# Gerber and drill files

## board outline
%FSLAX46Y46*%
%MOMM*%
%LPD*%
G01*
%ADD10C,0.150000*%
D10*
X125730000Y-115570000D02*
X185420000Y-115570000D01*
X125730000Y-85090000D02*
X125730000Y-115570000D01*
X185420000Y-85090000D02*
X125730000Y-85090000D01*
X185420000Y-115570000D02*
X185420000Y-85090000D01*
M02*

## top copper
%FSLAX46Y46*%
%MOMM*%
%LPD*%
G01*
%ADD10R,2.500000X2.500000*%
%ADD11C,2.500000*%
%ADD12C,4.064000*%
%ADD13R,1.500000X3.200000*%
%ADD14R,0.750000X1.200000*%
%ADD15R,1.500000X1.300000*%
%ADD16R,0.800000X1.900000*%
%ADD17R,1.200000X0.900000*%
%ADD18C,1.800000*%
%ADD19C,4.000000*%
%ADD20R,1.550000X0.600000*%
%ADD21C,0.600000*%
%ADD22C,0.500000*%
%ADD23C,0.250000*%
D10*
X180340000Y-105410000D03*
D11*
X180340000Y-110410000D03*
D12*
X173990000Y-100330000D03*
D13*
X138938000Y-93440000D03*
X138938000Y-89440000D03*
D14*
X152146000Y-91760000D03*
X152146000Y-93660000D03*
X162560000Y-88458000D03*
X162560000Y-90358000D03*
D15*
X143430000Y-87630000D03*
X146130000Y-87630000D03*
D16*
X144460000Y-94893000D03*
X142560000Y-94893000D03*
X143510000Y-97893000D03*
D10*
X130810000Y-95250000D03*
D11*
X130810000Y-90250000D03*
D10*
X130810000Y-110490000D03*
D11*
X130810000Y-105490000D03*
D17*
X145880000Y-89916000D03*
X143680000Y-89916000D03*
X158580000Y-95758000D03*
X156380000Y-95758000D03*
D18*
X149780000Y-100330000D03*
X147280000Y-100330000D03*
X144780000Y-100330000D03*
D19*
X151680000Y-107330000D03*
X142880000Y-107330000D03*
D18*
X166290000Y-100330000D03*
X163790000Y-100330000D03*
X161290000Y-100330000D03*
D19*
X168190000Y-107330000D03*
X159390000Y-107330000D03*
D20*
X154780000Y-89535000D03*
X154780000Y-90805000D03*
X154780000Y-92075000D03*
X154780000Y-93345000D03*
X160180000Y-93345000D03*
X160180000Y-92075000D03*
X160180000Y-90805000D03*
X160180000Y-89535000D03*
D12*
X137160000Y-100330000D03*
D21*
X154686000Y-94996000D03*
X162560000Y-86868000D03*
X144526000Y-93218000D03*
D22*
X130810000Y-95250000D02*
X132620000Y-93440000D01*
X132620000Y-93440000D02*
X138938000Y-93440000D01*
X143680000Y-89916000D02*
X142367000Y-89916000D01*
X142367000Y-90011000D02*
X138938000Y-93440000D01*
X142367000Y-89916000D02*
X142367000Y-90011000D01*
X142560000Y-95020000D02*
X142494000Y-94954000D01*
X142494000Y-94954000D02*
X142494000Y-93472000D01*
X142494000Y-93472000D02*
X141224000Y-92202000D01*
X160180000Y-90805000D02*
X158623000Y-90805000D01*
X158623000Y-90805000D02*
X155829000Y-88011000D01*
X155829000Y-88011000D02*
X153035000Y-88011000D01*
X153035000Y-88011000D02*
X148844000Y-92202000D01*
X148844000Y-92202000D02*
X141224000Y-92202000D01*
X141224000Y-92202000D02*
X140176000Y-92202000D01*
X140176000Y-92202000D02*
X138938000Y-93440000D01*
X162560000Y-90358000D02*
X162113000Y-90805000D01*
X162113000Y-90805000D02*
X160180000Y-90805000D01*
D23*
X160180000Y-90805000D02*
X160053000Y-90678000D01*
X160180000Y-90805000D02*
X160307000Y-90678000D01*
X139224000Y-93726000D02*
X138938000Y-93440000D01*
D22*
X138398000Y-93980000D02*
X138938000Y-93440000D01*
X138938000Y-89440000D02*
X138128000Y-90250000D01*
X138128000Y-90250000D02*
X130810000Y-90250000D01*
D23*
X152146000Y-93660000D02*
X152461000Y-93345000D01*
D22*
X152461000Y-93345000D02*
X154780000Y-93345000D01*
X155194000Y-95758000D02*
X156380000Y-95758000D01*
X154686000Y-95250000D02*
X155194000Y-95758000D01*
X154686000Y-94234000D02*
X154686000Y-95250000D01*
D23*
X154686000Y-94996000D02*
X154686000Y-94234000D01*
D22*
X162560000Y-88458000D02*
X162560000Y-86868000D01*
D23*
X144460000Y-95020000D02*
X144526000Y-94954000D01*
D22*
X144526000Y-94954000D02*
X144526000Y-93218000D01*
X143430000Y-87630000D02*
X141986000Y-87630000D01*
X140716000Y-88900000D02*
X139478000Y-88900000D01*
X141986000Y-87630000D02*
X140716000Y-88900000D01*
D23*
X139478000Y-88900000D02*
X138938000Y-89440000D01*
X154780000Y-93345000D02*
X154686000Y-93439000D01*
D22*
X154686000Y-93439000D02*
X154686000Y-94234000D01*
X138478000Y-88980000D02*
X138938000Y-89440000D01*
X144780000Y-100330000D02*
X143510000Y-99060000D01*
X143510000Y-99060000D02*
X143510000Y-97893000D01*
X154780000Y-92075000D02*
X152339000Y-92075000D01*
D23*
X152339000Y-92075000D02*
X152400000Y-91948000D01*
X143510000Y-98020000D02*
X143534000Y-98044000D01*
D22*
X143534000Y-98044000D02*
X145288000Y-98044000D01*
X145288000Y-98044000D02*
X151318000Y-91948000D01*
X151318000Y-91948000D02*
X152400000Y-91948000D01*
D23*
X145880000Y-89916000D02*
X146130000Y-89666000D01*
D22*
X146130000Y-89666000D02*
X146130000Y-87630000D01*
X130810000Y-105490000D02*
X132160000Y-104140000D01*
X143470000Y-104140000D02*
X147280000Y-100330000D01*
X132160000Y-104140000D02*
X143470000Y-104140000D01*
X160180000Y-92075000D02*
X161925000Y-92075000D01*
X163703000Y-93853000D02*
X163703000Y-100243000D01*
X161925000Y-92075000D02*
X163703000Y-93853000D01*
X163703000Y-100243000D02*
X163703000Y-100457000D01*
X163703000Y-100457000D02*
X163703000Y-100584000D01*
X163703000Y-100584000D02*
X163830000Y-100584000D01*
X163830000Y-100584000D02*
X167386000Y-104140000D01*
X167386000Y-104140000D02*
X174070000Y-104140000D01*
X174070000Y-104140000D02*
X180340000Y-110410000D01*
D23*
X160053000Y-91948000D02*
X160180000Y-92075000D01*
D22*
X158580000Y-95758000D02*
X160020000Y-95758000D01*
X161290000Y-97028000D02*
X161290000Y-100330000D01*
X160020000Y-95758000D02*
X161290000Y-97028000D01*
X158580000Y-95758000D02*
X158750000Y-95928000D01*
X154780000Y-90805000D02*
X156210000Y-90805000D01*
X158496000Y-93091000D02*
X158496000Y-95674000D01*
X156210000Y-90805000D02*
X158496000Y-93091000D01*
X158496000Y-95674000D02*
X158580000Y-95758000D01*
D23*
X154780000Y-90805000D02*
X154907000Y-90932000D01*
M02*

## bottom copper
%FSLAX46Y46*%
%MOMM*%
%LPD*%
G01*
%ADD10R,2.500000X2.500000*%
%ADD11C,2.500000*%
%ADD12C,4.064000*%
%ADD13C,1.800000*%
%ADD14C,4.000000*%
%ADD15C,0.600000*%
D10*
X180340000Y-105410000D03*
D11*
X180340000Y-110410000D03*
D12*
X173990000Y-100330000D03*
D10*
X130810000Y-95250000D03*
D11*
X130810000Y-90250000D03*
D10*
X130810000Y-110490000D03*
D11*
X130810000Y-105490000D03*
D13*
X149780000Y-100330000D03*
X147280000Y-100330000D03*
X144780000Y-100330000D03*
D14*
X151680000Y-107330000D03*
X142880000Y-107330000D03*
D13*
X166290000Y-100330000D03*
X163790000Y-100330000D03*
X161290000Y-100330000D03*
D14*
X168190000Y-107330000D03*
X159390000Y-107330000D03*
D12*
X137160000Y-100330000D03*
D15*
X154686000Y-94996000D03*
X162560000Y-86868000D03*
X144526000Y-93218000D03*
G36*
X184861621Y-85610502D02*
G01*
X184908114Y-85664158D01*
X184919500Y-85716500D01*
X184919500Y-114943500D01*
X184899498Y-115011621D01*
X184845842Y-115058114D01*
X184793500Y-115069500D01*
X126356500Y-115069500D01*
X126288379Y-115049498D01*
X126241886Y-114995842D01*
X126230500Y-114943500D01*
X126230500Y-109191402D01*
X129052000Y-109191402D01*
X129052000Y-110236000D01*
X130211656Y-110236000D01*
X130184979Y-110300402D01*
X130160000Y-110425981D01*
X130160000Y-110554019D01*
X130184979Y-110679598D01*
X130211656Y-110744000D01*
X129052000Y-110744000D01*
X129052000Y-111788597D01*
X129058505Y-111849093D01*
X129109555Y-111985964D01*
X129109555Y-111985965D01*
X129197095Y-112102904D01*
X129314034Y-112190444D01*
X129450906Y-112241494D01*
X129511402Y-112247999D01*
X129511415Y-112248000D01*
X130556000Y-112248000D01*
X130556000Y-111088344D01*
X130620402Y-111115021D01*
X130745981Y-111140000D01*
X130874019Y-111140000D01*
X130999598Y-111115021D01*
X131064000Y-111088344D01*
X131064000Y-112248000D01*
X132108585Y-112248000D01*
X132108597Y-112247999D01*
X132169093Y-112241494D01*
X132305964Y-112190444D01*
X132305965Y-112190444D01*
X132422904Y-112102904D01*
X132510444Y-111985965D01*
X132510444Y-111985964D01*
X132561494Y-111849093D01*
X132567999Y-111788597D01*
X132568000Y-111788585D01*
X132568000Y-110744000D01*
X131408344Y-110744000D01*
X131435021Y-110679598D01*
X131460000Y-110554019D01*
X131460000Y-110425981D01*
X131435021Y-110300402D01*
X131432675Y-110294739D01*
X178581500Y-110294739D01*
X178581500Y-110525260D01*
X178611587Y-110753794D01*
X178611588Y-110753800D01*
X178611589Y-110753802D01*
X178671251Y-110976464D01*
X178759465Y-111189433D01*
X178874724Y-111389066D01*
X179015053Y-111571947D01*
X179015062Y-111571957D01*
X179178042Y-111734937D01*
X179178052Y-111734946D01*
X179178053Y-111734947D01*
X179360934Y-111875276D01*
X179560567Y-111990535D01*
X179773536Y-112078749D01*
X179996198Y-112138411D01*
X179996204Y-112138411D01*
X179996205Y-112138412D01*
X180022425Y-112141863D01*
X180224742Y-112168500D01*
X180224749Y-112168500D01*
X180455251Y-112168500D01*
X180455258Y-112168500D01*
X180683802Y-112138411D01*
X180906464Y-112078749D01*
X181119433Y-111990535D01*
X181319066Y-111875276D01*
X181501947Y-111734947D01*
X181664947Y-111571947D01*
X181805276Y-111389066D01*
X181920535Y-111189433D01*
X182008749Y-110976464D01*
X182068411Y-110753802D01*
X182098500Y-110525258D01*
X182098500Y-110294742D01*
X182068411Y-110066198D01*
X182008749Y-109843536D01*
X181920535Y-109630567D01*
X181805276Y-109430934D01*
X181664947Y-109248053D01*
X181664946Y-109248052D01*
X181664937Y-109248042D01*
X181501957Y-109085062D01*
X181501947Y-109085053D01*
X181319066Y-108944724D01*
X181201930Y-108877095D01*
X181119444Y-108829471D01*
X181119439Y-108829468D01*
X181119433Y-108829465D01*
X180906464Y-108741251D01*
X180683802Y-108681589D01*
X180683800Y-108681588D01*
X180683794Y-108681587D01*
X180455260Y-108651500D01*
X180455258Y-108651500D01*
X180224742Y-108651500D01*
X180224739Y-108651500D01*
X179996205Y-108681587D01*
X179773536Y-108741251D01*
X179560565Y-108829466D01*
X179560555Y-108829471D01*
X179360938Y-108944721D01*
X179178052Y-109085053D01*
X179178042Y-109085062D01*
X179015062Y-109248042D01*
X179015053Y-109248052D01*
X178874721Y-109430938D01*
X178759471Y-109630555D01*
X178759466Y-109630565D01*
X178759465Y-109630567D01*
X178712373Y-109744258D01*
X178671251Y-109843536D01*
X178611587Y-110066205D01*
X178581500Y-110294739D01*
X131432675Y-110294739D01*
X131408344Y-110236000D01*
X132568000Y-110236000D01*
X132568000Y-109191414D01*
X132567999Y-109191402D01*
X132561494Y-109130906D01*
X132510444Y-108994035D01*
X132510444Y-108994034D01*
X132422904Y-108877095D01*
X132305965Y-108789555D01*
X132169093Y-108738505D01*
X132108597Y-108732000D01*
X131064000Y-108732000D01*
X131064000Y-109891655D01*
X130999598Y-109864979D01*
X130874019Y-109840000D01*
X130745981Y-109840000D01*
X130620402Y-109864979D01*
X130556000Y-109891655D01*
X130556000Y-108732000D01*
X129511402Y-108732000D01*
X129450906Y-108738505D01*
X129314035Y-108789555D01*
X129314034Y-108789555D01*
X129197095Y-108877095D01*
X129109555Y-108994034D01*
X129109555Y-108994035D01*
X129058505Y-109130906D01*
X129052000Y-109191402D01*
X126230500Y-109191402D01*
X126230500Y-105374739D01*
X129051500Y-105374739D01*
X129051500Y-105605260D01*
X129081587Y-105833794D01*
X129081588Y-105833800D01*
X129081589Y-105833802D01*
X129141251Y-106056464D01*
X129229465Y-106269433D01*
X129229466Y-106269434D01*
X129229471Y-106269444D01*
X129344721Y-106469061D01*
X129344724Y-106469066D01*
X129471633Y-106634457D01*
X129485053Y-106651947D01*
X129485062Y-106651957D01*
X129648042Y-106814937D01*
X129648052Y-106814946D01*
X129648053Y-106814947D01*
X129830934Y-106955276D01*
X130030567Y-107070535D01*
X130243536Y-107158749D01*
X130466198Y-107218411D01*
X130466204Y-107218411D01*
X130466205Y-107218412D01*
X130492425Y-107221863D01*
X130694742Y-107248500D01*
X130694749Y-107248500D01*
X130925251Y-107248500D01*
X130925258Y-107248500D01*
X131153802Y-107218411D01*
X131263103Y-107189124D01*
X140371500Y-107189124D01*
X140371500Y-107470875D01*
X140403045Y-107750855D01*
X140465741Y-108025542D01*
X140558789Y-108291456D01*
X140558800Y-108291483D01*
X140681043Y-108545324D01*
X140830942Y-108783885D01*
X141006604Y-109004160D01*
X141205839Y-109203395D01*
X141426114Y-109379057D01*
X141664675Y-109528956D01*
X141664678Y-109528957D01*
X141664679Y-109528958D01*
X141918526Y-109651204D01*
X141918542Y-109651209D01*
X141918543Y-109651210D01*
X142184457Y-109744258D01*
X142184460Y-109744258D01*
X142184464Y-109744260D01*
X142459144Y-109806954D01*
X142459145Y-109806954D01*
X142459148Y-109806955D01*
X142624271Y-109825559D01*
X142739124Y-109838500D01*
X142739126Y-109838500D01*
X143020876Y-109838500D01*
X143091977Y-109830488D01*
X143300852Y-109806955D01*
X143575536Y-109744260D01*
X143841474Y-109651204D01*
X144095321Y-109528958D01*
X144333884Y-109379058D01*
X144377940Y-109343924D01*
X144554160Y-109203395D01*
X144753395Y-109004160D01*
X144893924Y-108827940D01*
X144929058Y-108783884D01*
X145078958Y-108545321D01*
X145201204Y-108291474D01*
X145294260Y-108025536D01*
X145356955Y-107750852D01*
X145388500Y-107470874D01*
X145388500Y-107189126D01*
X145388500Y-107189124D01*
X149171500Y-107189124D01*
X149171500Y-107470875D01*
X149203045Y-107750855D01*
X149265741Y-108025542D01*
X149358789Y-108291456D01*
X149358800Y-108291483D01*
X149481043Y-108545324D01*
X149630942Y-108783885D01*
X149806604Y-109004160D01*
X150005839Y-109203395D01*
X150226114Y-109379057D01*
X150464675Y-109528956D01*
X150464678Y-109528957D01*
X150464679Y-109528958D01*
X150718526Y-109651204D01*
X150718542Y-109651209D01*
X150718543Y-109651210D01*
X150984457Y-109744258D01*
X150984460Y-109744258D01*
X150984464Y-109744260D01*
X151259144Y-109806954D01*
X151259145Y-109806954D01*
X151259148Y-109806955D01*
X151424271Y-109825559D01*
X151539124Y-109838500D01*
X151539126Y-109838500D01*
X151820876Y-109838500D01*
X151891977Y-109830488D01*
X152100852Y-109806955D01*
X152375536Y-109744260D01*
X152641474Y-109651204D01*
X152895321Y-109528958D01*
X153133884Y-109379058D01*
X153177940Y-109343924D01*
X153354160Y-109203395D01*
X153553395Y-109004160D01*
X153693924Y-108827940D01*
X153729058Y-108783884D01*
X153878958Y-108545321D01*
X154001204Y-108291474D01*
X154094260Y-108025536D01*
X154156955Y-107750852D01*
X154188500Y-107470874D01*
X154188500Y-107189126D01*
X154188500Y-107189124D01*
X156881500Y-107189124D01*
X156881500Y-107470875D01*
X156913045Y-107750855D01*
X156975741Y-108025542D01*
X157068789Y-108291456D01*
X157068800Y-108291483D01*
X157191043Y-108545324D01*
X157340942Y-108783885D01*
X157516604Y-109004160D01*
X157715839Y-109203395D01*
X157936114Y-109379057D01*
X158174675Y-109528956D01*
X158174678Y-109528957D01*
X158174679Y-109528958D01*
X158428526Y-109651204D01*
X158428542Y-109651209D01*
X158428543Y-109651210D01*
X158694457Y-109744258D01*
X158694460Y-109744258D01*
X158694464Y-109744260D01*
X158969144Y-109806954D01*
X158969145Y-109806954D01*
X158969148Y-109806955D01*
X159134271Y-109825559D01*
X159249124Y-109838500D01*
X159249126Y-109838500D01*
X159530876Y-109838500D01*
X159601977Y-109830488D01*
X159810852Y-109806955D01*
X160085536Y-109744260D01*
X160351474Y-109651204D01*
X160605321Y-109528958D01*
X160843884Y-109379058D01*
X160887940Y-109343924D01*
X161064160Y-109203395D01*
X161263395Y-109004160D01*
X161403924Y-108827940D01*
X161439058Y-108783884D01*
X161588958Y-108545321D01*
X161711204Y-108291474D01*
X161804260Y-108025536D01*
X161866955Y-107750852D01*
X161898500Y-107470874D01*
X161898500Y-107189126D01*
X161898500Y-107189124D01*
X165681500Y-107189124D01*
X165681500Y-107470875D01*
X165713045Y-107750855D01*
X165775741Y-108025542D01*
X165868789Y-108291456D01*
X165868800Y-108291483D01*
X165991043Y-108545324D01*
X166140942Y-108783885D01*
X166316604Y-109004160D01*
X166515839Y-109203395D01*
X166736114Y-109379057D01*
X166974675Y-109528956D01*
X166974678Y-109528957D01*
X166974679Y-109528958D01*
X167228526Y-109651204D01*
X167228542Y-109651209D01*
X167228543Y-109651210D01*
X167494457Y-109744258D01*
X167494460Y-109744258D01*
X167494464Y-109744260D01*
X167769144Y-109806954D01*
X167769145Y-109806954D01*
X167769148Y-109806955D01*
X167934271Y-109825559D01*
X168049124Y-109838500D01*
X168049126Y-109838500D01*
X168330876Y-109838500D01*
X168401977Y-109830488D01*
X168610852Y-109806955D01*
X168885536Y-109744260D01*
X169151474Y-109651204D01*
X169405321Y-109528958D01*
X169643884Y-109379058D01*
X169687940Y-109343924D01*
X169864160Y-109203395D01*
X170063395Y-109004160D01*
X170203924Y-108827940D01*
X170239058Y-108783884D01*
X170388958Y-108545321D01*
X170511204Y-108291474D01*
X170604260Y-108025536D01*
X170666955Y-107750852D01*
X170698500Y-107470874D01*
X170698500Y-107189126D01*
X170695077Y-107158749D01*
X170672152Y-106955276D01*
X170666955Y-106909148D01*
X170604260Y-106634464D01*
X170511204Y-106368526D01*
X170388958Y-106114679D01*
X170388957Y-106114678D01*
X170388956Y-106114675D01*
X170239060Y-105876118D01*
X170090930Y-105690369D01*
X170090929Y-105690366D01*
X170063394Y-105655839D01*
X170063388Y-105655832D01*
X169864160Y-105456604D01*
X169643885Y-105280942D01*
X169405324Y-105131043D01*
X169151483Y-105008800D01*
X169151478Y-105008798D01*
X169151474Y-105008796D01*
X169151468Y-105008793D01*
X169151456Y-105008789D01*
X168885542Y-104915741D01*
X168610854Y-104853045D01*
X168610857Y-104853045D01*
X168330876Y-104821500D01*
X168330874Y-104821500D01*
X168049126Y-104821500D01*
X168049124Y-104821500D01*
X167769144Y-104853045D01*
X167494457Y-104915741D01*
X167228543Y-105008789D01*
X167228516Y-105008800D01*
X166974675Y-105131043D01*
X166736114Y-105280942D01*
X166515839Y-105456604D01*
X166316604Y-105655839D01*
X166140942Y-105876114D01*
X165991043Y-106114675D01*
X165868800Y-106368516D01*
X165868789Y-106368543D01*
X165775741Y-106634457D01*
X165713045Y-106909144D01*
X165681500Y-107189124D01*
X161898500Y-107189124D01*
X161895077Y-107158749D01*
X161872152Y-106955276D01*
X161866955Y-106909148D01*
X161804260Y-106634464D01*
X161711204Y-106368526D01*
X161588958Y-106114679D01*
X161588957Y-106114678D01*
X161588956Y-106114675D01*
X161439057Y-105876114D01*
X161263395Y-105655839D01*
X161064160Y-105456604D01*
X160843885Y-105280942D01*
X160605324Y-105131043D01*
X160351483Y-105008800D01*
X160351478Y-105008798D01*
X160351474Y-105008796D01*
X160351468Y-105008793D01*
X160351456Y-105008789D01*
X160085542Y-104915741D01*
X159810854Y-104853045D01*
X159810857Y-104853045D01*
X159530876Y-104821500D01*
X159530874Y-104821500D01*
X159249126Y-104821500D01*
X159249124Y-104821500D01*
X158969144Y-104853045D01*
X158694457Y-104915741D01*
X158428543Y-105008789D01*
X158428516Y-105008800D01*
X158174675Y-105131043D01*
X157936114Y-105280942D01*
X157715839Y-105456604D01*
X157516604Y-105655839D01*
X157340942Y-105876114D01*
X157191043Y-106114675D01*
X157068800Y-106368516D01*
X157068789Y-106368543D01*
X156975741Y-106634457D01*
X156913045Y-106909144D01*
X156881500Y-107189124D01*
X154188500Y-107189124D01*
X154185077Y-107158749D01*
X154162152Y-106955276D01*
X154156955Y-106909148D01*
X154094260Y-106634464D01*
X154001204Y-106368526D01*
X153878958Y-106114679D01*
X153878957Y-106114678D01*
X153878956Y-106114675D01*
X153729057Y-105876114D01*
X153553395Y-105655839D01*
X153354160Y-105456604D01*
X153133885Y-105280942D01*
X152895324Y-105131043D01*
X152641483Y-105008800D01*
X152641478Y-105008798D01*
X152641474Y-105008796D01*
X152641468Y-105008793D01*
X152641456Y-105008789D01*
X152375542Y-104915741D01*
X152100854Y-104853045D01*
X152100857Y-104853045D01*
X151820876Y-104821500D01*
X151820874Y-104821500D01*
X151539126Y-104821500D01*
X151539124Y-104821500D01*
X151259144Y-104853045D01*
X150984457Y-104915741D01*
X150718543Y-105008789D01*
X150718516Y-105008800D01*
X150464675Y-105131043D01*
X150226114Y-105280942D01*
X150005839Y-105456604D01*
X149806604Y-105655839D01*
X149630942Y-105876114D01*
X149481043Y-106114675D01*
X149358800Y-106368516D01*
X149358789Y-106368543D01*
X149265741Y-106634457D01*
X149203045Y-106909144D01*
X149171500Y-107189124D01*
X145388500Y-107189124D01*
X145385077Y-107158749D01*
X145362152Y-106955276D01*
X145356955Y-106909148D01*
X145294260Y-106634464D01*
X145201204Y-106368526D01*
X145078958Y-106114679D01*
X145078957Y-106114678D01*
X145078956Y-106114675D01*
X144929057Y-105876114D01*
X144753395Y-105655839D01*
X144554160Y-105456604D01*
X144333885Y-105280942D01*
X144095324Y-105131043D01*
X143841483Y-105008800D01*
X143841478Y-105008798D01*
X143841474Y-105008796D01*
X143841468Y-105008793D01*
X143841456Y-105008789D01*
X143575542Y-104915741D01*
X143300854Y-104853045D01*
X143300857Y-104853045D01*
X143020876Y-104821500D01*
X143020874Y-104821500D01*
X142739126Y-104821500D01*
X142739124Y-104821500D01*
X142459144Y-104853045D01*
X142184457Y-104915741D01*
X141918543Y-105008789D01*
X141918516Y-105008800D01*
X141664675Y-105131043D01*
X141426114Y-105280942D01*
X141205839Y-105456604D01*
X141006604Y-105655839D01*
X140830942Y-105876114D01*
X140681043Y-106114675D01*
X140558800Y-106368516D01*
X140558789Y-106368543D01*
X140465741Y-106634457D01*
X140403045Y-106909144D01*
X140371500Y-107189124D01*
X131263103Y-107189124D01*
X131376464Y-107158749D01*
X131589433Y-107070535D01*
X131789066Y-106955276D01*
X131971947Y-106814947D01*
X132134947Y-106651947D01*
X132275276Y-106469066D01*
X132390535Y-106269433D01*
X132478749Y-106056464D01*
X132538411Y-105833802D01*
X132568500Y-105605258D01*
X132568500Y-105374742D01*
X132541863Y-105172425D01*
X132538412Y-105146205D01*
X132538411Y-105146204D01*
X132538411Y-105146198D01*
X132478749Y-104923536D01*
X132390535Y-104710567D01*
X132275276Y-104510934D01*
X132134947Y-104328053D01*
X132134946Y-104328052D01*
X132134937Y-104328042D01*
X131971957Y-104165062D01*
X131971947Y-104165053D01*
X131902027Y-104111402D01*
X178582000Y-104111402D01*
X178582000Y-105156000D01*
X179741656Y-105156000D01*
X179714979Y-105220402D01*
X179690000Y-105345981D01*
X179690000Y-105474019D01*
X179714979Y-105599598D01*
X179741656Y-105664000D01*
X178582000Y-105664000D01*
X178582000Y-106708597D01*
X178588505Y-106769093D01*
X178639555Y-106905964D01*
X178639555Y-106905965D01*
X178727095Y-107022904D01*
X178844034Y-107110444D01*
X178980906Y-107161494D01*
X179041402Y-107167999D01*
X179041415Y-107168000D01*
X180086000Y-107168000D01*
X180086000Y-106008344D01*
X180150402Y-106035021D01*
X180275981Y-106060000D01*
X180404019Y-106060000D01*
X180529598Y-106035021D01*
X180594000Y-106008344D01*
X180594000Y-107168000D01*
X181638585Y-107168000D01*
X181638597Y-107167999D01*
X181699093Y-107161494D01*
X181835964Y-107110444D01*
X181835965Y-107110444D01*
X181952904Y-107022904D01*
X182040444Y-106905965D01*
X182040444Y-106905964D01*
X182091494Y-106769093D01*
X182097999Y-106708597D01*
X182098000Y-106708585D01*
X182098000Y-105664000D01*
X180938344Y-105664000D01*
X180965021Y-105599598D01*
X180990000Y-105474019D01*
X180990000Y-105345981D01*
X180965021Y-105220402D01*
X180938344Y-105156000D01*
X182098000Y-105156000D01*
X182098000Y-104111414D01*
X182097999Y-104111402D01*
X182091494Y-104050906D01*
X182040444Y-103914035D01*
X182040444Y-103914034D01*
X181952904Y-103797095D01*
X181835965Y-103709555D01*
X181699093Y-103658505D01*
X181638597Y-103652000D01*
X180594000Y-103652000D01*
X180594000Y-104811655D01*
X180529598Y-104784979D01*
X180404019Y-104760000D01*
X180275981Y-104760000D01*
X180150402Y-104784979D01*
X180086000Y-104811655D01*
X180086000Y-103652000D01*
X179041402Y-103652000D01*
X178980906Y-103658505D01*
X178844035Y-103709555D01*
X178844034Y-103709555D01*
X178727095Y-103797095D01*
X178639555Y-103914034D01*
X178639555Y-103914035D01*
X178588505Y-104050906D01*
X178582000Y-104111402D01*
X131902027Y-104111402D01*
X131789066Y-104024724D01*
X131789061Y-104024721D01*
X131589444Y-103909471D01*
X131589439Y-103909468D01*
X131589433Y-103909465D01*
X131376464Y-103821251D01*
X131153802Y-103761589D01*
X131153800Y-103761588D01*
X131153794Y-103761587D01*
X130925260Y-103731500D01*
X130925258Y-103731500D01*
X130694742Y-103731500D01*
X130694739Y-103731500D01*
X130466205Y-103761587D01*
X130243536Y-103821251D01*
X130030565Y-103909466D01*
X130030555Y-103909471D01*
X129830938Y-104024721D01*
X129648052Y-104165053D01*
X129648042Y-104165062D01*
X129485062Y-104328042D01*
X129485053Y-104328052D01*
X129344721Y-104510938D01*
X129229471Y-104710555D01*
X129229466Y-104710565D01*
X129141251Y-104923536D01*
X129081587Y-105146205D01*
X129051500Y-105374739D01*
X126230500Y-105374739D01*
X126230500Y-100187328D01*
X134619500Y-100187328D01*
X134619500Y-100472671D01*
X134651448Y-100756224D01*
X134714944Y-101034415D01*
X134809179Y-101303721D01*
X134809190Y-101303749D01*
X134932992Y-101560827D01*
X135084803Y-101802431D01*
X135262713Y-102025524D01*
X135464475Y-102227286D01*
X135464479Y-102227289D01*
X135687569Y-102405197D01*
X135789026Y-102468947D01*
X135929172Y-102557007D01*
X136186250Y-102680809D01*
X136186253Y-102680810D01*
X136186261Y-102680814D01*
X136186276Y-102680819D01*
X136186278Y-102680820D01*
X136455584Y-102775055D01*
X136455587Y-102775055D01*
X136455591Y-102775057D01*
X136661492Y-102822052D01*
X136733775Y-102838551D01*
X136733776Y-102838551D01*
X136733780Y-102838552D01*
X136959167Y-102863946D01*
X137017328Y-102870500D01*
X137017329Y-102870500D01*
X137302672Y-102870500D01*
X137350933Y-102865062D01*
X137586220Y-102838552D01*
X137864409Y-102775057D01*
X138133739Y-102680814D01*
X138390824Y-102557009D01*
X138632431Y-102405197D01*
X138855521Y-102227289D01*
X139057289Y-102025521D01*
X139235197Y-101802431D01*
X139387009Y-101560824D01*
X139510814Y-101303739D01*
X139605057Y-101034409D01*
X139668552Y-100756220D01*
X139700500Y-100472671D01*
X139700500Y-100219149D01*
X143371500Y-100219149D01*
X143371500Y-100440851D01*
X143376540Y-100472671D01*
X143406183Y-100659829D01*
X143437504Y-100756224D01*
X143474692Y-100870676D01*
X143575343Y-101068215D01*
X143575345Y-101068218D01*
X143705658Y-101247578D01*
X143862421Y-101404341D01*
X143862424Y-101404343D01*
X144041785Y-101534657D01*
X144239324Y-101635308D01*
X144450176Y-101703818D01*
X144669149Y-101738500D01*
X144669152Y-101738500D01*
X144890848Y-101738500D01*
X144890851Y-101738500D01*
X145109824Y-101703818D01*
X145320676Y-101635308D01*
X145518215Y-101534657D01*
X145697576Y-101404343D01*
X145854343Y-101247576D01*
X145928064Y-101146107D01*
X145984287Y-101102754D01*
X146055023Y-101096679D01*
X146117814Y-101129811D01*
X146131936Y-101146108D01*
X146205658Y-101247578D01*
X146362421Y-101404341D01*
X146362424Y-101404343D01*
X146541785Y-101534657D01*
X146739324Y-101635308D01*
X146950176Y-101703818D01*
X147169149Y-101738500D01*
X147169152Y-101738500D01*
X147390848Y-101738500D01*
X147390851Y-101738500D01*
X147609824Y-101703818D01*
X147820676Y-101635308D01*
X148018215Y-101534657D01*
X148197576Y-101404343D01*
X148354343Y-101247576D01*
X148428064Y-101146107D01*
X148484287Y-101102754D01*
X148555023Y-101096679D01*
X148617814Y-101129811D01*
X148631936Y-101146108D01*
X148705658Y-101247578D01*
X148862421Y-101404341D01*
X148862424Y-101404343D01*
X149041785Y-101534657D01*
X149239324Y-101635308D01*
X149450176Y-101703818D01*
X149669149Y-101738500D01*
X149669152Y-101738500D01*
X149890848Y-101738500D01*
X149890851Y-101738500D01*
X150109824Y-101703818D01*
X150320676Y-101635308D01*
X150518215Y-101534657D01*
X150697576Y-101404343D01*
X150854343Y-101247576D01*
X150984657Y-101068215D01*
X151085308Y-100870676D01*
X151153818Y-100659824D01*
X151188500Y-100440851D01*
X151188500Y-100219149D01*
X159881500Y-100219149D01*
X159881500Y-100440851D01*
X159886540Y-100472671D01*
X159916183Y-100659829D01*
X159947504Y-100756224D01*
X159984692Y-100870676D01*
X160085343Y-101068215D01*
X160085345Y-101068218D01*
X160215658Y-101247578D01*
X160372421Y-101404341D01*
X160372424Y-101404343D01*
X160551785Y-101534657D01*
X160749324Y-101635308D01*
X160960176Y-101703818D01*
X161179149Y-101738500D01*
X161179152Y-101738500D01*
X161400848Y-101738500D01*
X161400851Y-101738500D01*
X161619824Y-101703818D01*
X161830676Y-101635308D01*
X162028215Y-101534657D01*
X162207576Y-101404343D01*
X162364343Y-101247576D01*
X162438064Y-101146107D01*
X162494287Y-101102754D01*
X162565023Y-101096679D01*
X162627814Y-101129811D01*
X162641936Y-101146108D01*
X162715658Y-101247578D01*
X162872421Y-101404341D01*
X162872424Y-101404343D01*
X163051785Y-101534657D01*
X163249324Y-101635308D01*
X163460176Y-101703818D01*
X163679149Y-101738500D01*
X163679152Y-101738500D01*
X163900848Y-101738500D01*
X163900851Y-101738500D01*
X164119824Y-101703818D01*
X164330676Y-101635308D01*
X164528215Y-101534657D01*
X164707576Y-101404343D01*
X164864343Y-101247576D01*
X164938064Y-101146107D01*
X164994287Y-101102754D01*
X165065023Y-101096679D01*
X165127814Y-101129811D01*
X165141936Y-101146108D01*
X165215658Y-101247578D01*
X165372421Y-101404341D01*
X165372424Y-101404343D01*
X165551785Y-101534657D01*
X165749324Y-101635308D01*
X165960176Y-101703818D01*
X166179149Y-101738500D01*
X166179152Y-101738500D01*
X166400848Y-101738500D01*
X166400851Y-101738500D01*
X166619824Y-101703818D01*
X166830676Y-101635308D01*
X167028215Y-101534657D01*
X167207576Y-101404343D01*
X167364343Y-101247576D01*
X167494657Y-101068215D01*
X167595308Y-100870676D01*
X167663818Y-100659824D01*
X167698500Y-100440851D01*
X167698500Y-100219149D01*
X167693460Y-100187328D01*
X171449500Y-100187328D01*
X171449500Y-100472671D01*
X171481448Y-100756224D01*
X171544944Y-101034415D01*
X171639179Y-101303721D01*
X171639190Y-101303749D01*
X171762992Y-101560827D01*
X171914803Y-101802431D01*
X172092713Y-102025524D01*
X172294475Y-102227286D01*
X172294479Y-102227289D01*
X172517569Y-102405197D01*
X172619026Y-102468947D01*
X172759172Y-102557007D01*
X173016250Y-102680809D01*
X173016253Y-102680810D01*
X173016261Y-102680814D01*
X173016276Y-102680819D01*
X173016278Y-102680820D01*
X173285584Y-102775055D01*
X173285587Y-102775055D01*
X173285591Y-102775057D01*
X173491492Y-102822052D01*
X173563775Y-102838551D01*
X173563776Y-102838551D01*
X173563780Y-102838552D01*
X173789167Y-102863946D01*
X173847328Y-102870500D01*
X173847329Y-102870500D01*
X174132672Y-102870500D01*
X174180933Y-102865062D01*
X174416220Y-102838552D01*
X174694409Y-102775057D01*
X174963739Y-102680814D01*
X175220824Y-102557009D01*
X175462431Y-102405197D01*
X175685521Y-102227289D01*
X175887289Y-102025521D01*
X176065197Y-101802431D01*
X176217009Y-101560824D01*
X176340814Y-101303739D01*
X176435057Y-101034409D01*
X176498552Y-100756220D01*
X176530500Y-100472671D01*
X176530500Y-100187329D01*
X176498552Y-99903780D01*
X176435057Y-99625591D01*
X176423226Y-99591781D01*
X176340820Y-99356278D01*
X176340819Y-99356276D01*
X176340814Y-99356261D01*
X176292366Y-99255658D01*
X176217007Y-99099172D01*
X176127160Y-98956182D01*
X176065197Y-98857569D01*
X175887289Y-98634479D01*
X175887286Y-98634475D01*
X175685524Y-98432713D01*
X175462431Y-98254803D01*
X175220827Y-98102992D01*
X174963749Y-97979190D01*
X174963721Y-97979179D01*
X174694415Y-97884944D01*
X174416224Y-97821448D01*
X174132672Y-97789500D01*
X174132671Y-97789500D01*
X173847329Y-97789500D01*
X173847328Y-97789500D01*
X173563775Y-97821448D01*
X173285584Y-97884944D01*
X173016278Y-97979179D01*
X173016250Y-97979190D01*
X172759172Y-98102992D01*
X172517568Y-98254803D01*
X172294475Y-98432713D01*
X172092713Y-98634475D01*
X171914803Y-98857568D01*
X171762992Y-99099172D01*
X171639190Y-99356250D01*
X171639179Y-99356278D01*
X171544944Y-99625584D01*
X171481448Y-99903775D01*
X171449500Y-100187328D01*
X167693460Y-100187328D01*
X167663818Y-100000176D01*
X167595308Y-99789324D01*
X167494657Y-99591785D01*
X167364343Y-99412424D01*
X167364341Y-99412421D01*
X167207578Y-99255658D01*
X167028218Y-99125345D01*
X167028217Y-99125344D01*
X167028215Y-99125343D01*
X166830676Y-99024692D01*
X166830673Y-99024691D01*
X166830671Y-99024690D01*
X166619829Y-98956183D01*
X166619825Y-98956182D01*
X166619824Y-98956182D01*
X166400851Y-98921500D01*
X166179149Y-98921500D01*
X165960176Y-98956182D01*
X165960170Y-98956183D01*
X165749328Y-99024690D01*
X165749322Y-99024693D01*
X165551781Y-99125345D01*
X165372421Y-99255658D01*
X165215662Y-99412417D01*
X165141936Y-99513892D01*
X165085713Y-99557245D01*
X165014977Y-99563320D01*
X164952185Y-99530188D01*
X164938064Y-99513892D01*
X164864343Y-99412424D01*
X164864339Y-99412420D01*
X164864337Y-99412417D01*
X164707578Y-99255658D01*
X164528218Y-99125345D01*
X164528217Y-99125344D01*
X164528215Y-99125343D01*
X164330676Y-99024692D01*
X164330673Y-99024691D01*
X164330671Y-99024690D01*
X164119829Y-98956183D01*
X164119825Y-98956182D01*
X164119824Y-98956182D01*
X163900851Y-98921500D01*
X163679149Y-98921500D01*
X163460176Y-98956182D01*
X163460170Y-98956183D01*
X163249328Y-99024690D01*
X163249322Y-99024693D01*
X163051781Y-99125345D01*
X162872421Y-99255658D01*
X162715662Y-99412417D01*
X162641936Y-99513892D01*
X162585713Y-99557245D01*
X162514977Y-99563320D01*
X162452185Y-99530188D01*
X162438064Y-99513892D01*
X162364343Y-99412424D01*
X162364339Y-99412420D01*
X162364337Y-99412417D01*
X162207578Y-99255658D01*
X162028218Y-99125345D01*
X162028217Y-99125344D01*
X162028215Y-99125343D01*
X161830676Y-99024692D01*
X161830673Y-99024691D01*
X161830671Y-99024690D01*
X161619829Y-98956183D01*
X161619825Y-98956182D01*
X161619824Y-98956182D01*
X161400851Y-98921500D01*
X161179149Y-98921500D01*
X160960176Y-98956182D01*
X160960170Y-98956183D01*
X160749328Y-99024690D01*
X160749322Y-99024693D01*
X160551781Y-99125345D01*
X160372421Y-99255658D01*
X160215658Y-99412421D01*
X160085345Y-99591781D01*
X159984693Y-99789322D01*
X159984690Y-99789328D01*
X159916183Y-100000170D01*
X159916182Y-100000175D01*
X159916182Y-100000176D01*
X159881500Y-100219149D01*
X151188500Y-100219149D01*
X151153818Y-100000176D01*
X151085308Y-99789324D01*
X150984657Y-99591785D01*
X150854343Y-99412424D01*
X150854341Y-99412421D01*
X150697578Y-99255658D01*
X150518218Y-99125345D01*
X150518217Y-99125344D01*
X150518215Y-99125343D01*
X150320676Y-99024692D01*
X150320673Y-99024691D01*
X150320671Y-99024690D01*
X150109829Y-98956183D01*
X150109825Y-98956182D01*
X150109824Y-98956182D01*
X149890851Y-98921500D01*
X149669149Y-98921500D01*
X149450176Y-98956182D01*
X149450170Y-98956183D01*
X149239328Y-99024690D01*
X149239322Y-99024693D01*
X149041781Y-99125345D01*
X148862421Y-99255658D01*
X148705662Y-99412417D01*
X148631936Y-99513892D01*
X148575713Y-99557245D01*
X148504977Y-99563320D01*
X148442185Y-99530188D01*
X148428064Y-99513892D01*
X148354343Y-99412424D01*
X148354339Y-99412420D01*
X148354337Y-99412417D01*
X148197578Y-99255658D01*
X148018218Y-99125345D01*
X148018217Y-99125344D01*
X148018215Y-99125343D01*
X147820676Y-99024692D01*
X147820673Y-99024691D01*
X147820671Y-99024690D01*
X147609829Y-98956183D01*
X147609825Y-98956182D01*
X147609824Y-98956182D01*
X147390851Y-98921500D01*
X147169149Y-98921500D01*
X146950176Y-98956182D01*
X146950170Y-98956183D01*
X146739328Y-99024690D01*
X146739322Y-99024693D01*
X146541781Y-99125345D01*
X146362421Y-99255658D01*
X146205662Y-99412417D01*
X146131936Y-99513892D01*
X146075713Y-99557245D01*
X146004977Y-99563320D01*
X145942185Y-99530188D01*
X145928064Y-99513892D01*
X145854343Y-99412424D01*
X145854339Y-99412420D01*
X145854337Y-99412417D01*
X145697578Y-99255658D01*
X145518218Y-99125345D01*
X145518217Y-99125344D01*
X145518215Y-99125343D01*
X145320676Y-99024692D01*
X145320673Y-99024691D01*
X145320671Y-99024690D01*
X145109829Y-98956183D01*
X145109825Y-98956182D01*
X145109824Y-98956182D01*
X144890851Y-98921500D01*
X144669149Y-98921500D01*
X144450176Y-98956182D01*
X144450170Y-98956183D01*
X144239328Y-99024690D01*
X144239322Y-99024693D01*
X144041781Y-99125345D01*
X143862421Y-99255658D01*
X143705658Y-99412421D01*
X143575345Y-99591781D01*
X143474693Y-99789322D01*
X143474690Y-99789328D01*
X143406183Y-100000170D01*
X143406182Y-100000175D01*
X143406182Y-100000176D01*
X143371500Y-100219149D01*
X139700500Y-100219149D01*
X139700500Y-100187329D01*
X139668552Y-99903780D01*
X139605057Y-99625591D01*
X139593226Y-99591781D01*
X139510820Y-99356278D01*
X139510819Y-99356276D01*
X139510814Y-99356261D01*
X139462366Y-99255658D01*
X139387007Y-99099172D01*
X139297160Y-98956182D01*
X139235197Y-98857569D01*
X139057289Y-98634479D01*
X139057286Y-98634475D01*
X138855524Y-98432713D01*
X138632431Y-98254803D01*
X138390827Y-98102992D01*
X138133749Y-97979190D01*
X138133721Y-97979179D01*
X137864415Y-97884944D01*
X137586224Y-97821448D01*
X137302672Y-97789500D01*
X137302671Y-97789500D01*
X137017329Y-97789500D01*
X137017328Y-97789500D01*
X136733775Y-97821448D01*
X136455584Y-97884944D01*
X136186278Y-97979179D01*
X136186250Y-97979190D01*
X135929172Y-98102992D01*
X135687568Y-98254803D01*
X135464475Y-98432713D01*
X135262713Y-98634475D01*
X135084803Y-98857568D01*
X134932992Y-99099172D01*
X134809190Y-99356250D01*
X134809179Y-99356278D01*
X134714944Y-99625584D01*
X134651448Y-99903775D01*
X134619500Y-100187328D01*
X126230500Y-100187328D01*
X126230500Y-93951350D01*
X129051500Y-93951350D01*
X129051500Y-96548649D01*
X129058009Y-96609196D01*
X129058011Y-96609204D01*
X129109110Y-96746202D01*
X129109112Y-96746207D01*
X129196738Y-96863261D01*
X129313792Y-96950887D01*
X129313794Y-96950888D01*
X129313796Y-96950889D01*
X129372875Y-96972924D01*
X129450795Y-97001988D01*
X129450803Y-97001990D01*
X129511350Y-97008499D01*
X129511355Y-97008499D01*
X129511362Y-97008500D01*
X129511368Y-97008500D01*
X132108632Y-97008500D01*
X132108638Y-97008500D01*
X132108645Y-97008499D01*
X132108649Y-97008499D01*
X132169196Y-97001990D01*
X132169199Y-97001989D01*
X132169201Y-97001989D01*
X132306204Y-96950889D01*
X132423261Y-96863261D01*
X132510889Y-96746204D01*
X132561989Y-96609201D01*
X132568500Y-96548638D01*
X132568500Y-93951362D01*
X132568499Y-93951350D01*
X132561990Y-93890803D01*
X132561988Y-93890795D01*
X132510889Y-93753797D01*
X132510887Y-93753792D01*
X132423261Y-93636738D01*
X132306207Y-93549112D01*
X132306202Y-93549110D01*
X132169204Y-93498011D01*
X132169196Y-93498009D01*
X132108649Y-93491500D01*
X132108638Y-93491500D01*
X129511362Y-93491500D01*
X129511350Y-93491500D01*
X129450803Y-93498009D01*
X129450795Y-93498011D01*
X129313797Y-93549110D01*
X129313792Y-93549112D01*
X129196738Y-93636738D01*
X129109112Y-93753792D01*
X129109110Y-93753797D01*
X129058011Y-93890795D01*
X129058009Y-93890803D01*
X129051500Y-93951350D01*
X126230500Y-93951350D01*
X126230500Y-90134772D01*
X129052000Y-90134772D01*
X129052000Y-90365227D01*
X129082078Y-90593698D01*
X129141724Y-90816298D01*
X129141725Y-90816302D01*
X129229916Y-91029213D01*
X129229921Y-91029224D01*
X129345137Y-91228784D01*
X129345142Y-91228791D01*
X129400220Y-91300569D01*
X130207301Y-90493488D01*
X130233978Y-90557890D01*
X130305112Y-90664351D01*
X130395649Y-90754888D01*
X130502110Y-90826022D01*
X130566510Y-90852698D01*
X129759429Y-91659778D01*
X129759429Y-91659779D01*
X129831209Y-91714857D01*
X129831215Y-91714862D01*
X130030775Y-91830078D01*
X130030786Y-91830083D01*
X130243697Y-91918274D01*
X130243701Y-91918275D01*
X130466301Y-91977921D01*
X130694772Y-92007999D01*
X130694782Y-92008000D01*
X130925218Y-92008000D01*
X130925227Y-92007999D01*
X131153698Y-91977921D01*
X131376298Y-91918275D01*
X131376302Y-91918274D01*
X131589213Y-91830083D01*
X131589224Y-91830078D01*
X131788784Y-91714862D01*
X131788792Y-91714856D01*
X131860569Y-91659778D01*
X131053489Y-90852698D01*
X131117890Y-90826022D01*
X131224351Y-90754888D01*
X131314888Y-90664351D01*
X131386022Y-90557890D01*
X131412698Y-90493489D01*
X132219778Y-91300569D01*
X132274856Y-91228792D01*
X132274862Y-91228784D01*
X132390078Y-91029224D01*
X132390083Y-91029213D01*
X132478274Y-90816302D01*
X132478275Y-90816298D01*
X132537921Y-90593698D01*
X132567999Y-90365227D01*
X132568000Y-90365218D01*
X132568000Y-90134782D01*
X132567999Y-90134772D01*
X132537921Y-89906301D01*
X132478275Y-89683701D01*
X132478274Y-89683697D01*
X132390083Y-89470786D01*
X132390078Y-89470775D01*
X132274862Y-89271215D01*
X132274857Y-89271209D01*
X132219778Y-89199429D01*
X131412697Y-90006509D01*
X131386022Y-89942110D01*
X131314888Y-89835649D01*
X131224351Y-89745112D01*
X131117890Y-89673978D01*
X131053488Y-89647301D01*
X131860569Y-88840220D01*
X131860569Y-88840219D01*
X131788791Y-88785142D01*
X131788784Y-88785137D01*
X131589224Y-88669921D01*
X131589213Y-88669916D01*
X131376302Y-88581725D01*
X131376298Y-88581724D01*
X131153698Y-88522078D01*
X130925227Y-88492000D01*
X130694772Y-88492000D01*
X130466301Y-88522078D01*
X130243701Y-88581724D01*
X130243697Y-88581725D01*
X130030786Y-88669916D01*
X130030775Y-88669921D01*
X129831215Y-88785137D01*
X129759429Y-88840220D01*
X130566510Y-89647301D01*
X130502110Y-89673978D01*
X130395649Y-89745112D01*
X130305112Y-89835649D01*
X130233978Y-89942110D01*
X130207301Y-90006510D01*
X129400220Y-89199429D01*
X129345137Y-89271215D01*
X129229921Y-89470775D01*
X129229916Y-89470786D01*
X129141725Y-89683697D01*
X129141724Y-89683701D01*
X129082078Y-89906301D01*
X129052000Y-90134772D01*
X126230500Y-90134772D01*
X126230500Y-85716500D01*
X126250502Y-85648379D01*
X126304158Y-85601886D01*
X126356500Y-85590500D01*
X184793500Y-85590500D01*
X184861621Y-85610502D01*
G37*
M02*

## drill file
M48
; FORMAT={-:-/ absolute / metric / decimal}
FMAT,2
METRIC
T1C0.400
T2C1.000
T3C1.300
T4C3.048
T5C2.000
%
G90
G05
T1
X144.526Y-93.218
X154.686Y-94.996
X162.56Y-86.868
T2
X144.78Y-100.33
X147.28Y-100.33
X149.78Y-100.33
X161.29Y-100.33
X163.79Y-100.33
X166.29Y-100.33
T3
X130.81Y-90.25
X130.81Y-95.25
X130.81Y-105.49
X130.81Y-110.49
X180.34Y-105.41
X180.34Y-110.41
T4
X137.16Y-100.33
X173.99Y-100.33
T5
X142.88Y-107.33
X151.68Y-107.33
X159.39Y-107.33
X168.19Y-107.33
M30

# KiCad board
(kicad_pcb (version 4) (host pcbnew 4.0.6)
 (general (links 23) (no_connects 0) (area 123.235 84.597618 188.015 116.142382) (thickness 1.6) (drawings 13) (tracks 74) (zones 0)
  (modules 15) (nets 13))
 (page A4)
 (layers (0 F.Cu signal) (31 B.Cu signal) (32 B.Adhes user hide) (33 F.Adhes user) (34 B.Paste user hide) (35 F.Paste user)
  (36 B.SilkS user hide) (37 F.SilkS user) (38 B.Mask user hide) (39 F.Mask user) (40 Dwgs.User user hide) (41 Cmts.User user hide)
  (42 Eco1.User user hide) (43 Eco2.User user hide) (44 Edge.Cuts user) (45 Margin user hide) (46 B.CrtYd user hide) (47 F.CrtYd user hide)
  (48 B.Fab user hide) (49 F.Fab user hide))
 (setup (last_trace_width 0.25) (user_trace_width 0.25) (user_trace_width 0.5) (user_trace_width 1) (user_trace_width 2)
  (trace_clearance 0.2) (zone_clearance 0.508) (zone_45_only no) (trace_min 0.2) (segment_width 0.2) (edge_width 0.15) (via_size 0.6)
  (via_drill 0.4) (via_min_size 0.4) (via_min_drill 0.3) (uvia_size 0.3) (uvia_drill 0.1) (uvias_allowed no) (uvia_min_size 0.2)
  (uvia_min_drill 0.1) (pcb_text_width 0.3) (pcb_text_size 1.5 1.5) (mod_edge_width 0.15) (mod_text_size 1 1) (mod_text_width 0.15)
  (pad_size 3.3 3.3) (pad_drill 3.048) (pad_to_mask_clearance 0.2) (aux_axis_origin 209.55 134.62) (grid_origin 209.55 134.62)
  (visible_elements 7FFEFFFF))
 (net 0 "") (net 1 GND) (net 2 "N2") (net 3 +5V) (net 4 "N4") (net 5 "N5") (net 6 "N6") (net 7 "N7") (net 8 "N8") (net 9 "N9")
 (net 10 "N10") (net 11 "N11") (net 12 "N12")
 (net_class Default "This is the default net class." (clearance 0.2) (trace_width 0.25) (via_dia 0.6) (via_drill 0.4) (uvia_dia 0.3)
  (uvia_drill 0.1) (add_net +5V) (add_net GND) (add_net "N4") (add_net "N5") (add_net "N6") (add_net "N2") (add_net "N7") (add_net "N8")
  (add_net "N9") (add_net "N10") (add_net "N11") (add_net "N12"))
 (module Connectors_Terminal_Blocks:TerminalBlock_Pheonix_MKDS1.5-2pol (layer F.Cu) (at 180.34 105.41 270)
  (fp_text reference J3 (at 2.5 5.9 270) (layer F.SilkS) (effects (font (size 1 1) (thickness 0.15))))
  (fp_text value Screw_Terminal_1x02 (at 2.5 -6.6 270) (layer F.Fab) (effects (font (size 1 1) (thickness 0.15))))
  (pad 1 thru_hole rect (at 0 0 270) (size 2.5 2.5) (drill 1.3) (layers *.Cu *.Mask) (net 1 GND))
  (pad 2 thru_hole circle (at 5 0 270) (size 2.5 2.5) (drill 1.3) (layers *.Cu *.Mask) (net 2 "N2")))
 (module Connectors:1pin (layer F.Cu) (at 173.99 100.33)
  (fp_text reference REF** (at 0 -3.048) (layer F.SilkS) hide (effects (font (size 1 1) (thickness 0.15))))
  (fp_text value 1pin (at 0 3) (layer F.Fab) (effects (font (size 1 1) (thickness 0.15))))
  (pad 1 thru_hole circle (at 0 0) (size 4.064 4.064) (drill 3.048) (layers *.Cu *.Mask)))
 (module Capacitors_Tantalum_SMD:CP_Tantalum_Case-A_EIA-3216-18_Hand (layer F.Cu) (at 138.938 91.44 90)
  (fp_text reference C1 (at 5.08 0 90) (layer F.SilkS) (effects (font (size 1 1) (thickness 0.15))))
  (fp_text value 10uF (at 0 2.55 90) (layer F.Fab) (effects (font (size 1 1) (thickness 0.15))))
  (pad 1 smd rect (at -2 0 90) (size 3.2 1.5) (layers F.Cu F.Paste F.Mask) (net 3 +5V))
  (pad 2 smd rect (at 2 0 90) (size 3.2 1.5) (layers F.Cu F.Paste F.Mask) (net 1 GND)))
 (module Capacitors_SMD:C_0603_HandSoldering (layer F.Cu) (at 152.146 92.71 270)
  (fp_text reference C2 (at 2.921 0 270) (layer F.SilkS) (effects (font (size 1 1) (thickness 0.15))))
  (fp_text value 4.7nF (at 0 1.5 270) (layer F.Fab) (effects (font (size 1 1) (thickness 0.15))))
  (pad 1 smd rect (at -0.95 0 270) (size 1.2 0.75) (layers F.Cu F.Paste F.Mask) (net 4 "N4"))
  (pad 2 smd rect (at 0.95 0 270) (size 1.2 0.75) (layers F.Cu F.Paste F.Mask) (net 1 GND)))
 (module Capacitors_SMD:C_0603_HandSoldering (layer F.Cu) (at 162.56 89.408 270)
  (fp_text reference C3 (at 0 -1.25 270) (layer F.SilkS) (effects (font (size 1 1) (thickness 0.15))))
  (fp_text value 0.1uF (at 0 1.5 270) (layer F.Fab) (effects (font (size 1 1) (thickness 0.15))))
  (pad 1 smd rect (at -0.95 0 270) (size 1.2 0.75) (layers F.Cu F.Paste F.Mask) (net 1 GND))
  (pad 2 smd rect (at 0.95 0 270) (size 1.2 0.75) (layers F.Cu F.Paste F.Mask) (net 3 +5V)))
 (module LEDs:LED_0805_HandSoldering (layer F.Cu) (at 144.78 87.63)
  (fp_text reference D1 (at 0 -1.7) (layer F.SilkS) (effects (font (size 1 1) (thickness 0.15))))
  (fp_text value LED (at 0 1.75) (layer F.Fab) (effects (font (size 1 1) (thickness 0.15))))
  (pad 1 smd rect (at -1.35 0) (size 1.5 1.3) (layers F.Cu F.Paste F.Mask) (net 1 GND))
  (pad 2 smd rect (at 1.35 0) (size 1.5 1.3) (layers F.Cu F.Paste F.Mask) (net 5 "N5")))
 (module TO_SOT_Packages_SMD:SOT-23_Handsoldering (layer F.Cu) (at 143.51 96.393 270)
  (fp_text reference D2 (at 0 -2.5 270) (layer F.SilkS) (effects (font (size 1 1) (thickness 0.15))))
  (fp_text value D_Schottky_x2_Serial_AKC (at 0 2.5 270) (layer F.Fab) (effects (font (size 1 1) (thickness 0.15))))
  (pad 1 smd rect (at -1.5 -0.95 270) (size 1.9 0.8) (layers F.Cu F.Paste F.Mask) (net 1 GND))
  (pad 2 smd rect (at -1.5 0.95 270) (size 1.9 0.8) (layers F.Cu F.Paste F.Mask) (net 3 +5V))
  (pad 3 smd rect (at 1.5 0 270) (size 1.9 0.8) (layers F.Cu F.Paste F.Mask) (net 4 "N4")))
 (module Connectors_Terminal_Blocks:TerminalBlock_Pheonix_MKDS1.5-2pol (layer F.Cu) (at 130.81 95.25 90)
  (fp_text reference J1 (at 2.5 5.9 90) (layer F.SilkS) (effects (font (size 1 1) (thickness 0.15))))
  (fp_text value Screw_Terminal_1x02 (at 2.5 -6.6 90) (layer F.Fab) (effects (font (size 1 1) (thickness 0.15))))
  (pad 1 thru_hole rect (at 0 0 90) (size 2.5 2.5) (drill 1.3) (layers *.Cu *.Mask) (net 3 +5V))
  (pad 2 thru_hole circle (at 5 0 90) (size 2.5 2.5) (drill 1.3) (layers *.Cu *.Mask) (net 1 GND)))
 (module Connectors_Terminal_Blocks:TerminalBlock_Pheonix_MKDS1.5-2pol (layer F.Cu) (at 130.81 110.49 90)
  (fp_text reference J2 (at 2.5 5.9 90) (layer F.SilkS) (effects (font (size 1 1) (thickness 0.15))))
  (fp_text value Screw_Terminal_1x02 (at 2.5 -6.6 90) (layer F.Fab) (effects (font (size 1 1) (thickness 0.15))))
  (pad 1 thru_hole rect (at 0 0 90) (size 2.5 2.5) (drill 1.3) (layers *.Cu *.Mask) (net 1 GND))
  (pad 2 thru_hole circle (at 5 0 90) (size 2.5 2.5) (drill 1.3) (layers *.Cu *.Mask) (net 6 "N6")))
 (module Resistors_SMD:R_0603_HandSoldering (layer F.Cu) (at 144.78 89.916 180)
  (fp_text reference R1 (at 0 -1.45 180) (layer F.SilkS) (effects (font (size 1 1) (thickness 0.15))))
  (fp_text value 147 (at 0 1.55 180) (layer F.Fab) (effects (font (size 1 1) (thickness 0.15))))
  (pad 1 smd rect (at -1.1 0 180) (size 1.2 0.9) (layers F.Cu F.Paste F.Mask) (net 5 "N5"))
  (pad 2 smd rect (at 1.1 0 180) (size 1.2 0.9) (layers F.Cu F.Paste F.Mask) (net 3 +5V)))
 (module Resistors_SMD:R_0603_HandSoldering (layer F.Cu) (at 157.48 95.758 180)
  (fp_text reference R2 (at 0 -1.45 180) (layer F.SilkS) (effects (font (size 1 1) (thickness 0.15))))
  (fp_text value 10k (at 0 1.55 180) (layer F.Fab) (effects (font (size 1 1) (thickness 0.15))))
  (pad 1 smd rect (at -1.1 0 180) (size 1.2 0.9) (layers F.Cu F.Paste F.Mask) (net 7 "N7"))
  (pad 2 smd rect (at 1.1 0 180) (size 1.2 0.9) (layers F.Cu F.Paste F.Mask) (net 1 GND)))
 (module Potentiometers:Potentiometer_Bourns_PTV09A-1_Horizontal (layer F.Cu) (at 144.78 100.33 270)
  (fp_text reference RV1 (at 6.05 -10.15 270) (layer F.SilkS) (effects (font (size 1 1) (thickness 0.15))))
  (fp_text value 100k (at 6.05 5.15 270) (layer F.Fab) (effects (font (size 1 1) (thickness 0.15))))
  (pad 3 thru_hole circle (at 0 -5 270) (size 1.8 1.8) (drill 1) (layers *.Cu *.Mask) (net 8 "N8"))
  (pad 2 thru_hole circle (at 0 -2.5 270) (size 1.8 1.8) (drill 1) (layers *.Cu *.Mask) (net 6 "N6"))
  (pad 1 thru_hole circle (at 0 0 270) (size 1.8 1.8) (drill 1) (layers *.Cu *.Mask) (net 4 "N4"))
  (pad 0 np_thru_hole circle (at 7 -6.9 270) (size 4 4) (drill 2) (layers *.Cu *.Mask))
  (pad 0 np_thru_hole circle (at 7 1.9 270) (size 4 4) (drill 2) (layers *.Cu *.Mask)))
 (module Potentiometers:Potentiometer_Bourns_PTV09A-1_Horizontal (layer F.Cu) (at 161.29 100.33 270)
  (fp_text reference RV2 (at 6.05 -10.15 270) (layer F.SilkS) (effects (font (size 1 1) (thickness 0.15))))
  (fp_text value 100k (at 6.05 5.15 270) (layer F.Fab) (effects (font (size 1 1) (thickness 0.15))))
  (pad 3 thru_hole circle (at 0 -5 270) (size 1.8 1.8) (drill 1) (layers *.Cu *.Mask) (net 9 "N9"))
  (pad 2 thru_hole circle (at 0 -2.5 270) (size 1.8 1.8) (drill 1) (layers *.Cu *.Mask) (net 2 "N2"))
  (pad 1 thru_hole circle (at 0 0 270) (size 1.8 1.8) (drill 1) (layers *.Cu *.Mask) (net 7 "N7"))
  (pad 0 np_thru_hole circle (at 7 -6.9 270) (size 4 4) (drill 2) (layers *.Cu *.Mask))
  (pad 0 np_thru_hole circle (at 7 1.9 270) (size 4 4) (drill 2) (layers *.Cu *.Mask)))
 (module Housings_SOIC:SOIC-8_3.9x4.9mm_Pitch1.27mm (layer F.Cu) (at 157.48 91.44)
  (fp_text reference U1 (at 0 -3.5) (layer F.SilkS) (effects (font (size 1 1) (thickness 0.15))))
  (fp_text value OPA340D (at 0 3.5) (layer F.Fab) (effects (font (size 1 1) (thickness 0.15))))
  (pad 1 smd rect (at -2.7 -1.905) (size 1.55 0.6) (layers F.Cu F.Paste F.Mask) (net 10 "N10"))
  (pad 2 smd rect (at -2.7 -0.635) (size 1.55 0.6) (layers F.Cu F.Paste F.Mask) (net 7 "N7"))
  (pad 3 smd rect (at -2.7 0.635) (size 1.55 0.6) (layers F.Cu F.Paste F.Mask) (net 4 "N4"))
  (pad 4 smd rect (at -2.7 1.905) (size 1.55 0.6) (layers F.Cu F.Paste F.Mask) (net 1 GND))
  (pad 5 smd rect (at 2.7 1.905) (size 1.55 0.6) (layers F.Cu F.Paste F.Mask) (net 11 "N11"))
  (pad 6 smd rect (at 2.7 0.635) (size 1.55 0.6) (layers F.Cu F.Paste F.Mask) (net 2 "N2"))
  (pad 7 smd rect (at 2.7 -0.635) (size 1.55 0.6) (layers F.Cu F.Paste F.Mask) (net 3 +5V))
  (pad 8 smd rect (at 2.7 -1.905) (size 1.55 0.6) (layers F.Cu F.Paste F.Mask) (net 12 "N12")))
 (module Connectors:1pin (layer F.Cu) (at 137.16 100.33)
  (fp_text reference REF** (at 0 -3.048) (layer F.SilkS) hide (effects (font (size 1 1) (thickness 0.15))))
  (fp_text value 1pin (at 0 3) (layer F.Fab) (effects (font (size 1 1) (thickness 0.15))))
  (pad 1 thru_hole circle (at 0 0) (size 4.064 4.064) (drill 3.048) (layers *.Cu *.Mask)))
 (gr_line (start 125.73 115.57) (end 185.42 115.57) (angle 90) (layer Edge.Cuts) (width 0.15))
 (gr_line (start 125.73 85.09) (end 125.73 115.57) (angle 90) (layer Edge.Cuts) (width 0.15))
 (gr_line (start 185.42 85.09) (end 125.73 85.09) (angle 90) (layer Edge.Cuts) (width 0.15))
 (gr_line (start 185.42 115.57) (end 185.42 85.09) (angle 90) (layer Edge.Cuts) (width 0.15))
 (segment (start 130.81 95.25) (end 132.62 93.44) (width 0.5) (layer F.Cu) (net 3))
 (segment (start 132.62 93.44) (end 138.938 93.44) (width 0.5) (layer F.Cu) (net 3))
 (segment (start 143.68 89.916) (end 142.367 89.916) (width 0.5) (layer F.Cu) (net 3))
 (segment (start 142.367 90.011) (end 138.938 93.44) (width 0.5) (layer F.Cu) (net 3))
 (segment (start 142.367 89.916) (end 142.367 90.011) (width 0.5) (layer F.Cu) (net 3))
 (segment (start 142.56 95.02) (end 142.494 94.954) (width 0.5) (layer F.Cu) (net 3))
 (segment (start 142.494 94.954) (end 142.494 93.472) (width 0.5) (layer F.Cu) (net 3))
 (segment (start 142.494 93.472) (end 141.224 92.202) (width 0.5) (layer F.Cu) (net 3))
 (segment (start 160.18 90.805) (end 158.623 90.805) (width 0.5) (layer F.Cu) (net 3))
 (segment (start 158.623 90.805) (end 155.829 88.011) (width 0.5) (layer F.Cu) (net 3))
 (segment (start 155.829 88.011) (end 153.035 88.011) (width 0.5) (layer F.Cu) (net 3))
 (segment (start 153.035 88.011) (end 148.844 92.202) (width 0.5) (layer F.Cu) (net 3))
 (segment (start 148.844 92.202) (end 141.224 92.202) (width 0.5) (layer F.Cu) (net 3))
 (segment (start 141.224 92.202) (end 140.176 92.202) (width 0.5) (layer F.Cu) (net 3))
 (segment (start 140.176 92.202) (end 138.938 93.44) (width 0.5) (layer F.Cu) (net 3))
 (segment (start 162.56 90.358) (end 162.113 90.805) (width 0.5) (layer F.Cu) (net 3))
 (segment (start 162.113 90.805) (end 160.18 90.805) (width 0.5) (layer F.Cu) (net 3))
 (segment (start 160.18 90.805) (end 160.053 90.678) (width 0.25) (layer F.Cu) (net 3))
 (segment (start 160.18 90.805) (end 160.307 90.678) (width 0.25) (layer F.Cu) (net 3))
 (segment (start 139.224 93.726) (end 138.938 93.44) (width 0.25) (layer F.Cu) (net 3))
 (segment (start 138.398 93.98) (end 138.938 93.44) (width 0.5) (layer F.Cu) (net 3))
 (segment (start 138.938 89.44) (end 138.128 90.25) (width 0.5) (layer F.Cu) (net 1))
 (segment (start 138.128 90.25) (end 130.81 90.25) (width 0.5) (layer F.Cu) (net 1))
 (segment (start 152.146 93.66) (end 152.461 93.345) (width 0.25) (layer F.Cu) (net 1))
 (segment (start 152.461 93.345) (end 154.78 93.345) (width 0.5) (layer F.Cu) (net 1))
 (via (at 154.686 94.996) (size 0.6) (drill 0.4) (layers F.Cu B.Cu) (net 1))
 (segment (start 155.194 95.758) (end 156.38 95.758) (width 0.5) (layer F.Cu) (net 1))
 (segment (start 154.686 95.25) (end 155.194 95.758) (width 0.5) (layer F.Cu) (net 1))
 (segment (start 154.686 94.234) (end 154.686 95.25) (width 0.5) (layer F.Cu) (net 1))
 (segment (start 154.686 94.996) (end 154.686 94.234) (width 0.25) (layer F.Cu) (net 1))
 (segment (start 162.56 88.458) (end 162.56 86.868) (width 0.5) (layer F.Cu) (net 1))
 (via (at 162.56 86.868) (size 0.6) (drill 0.4) (layers F.Cu B.Cu) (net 1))
 (segment (start 144.46 95.02) (end 144.526 94.954) (width 0.25) (layer F.Cu) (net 1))
 (segment (start 144.526 94.954) (end 144.526 93.218) (width 0.5) (layer F.Cu) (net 1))
 (via (at 144.526 93.218) (size 0.6) (drill 0.4) (layers F.Cu B.Cu) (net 1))
 (segment (start 143.43 87.63) (end 141.986 87.63) (width 0.5) (layer F.Cu) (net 1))
 (segment (start 140.716 88.9) (end 139.478 88.9) (width 0.5) (layer F.Cu) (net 1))
 (segment (start 141.986 87.63) (end 140.716 88.9) (width 0.5) (layer F.Cu) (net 1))
 (segment (start 139.478 88.9) (end 138.938 89.44) (width 0.25) (layer F.Cu) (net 1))
 (segment (start 154.78 93.345) (end 154.686 93.439) (width 0.25) (layer F.Cu) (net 1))
 (segment (start 154.686 93.439) (end 154.686 94.234) (width 0.5) (layer F.Cu) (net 1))
 (segment (start 138.478 88.98) (end 138.938 89.44) (width 0.5) (layer F.Cu) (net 1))
 (segment (start 144.78 100.33) (end 143.51 99.06) (width 0.5) (layer F.Cu) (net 4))
 (segment (start 143.51 99.06) (end 143.51 97.893) (width 0.5) (layer F.Cu) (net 4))
 (segment (start 154.78 92.075) (end 152.339 92.075) (width 0.5) (layer F.Cu) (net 4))
 (segment (start 152.339 92.075) (end 152.4 91.948) (width 0.25) (layer F.Cu) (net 4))
 (segment (start 143.51 98.02) (end 143.534 98.044) (width 0.25) (layer F.Cu) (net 4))
 (segment (start 143.534 98.044) (end 145.288 98.044) (width 0.5) (layer F.Cu) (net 4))
 (segment (start 145.288 98.044) (end 151.318 91.948) (width 0.5) (layer F.Cu) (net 4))
 (segment (start 151.318 91.948) (end 152.4 91.948) (width 0.5) (layer F.Cu) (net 4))
 (segment (start 145.88 89.916) (end 146.13 89.666) (width 0.25) (layer F.Cu) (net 5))
 (segment (start 146.13 89.666) (end 146.13 87.63) (width 0.5) (layer F.Cu) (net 5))
 (segment (start 130.81 105.49) (end 132.16 104.14) (width 0.5) (layer F.Cu) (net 6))
 (segment (start 143.47 104.14) (end 147.28 100.33) (width 0.5) (layer F.Cu) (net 6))
 (segment (start 132.16 104.14) (end 143.47 104.14) (width 0.5) (layer F.Cu) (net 6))
 (segment (start 160.18 92.075) (end 161.925 92.075) (width 0.5) (layer F.Cu) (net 2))
 (segment (start 163.703 93.853) (end 163.703 100.243) (width 0.5) (layer F.Cu) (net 2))
 (segment (start 161.925 92.075) (end 163.703 93.853) (width 0.5) (layer F.Cu) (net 2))
 (segment (start 163.703 100.243) (end 163.703 100.457) (width 0.5) (layer F.Cu) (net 2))
 (segment (start 163.703 100.457) (end 163.703 100.584) (width 0.5) (layer F.Cu) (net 2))
 (segment (start 163.703 100.584) (end 163.83 100.584) (width 0.5) (layer F.Cu) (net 2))
 (segment (start 163.83 100.584) (end 167.386 104.14) (width 0.5) (layer F.Cu) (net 2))
 (segment (start 167.386 104.14) (end 174.07 104.14) (width 0.5) (layer F.Cu) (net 2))
 (segment (start 174.07 104.14) (end 180.34 110.41) (width 0.5) (layer F.Cu) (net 2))
 (segment (start 160.053 91.948) (end 160.18 92.075) (width 0.25) (layer F.Cu) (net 2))
 (segment (start 158.58 95.758) (end 160.02 95.758) (width 0.5) (layer F.Cu) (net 7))
 (segment (start 161.29 97.028) (end 161.29 100.33) (width 0.5) (layer F.Cu) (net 7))
 (segment (start 160.02 95.758) (end 161.29 97.028) (width 0.5) (layer F.Cu) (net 7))
 (segment (start 158.58 95.758) (end 158.75 95.928) (width 0.5) (layer F.Cu) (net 7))
 (segment (start 154.78 90.805) (end 156.21 90.805) (width 0.5) (layer F.Cu) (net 7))
 (segment (start 158.496 93.091) (end 158.496 95.674) (width 0.5) (layer F.Cu) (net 7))
 (segment (start 156.21 90.805) (end 158.496 93.091) (width 0.5) (layer F.Cu) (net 7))
 (segment (start 158.496 95.674) (end 158.58 95.758) (width 0.5) (layer F.Cu) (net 7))
 (segment (start 154.78 90.805) (end 154.907 90.932) (width 0.25) (layer F.Cu) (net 7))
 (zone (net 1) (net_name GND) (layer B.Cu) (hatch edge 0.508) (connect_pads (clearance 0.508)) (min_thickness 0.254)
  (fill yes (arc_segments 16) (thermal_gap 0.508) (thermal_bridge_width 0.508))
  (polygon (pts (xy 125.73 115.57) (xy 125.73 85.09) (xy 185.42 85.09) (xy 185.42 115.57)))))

